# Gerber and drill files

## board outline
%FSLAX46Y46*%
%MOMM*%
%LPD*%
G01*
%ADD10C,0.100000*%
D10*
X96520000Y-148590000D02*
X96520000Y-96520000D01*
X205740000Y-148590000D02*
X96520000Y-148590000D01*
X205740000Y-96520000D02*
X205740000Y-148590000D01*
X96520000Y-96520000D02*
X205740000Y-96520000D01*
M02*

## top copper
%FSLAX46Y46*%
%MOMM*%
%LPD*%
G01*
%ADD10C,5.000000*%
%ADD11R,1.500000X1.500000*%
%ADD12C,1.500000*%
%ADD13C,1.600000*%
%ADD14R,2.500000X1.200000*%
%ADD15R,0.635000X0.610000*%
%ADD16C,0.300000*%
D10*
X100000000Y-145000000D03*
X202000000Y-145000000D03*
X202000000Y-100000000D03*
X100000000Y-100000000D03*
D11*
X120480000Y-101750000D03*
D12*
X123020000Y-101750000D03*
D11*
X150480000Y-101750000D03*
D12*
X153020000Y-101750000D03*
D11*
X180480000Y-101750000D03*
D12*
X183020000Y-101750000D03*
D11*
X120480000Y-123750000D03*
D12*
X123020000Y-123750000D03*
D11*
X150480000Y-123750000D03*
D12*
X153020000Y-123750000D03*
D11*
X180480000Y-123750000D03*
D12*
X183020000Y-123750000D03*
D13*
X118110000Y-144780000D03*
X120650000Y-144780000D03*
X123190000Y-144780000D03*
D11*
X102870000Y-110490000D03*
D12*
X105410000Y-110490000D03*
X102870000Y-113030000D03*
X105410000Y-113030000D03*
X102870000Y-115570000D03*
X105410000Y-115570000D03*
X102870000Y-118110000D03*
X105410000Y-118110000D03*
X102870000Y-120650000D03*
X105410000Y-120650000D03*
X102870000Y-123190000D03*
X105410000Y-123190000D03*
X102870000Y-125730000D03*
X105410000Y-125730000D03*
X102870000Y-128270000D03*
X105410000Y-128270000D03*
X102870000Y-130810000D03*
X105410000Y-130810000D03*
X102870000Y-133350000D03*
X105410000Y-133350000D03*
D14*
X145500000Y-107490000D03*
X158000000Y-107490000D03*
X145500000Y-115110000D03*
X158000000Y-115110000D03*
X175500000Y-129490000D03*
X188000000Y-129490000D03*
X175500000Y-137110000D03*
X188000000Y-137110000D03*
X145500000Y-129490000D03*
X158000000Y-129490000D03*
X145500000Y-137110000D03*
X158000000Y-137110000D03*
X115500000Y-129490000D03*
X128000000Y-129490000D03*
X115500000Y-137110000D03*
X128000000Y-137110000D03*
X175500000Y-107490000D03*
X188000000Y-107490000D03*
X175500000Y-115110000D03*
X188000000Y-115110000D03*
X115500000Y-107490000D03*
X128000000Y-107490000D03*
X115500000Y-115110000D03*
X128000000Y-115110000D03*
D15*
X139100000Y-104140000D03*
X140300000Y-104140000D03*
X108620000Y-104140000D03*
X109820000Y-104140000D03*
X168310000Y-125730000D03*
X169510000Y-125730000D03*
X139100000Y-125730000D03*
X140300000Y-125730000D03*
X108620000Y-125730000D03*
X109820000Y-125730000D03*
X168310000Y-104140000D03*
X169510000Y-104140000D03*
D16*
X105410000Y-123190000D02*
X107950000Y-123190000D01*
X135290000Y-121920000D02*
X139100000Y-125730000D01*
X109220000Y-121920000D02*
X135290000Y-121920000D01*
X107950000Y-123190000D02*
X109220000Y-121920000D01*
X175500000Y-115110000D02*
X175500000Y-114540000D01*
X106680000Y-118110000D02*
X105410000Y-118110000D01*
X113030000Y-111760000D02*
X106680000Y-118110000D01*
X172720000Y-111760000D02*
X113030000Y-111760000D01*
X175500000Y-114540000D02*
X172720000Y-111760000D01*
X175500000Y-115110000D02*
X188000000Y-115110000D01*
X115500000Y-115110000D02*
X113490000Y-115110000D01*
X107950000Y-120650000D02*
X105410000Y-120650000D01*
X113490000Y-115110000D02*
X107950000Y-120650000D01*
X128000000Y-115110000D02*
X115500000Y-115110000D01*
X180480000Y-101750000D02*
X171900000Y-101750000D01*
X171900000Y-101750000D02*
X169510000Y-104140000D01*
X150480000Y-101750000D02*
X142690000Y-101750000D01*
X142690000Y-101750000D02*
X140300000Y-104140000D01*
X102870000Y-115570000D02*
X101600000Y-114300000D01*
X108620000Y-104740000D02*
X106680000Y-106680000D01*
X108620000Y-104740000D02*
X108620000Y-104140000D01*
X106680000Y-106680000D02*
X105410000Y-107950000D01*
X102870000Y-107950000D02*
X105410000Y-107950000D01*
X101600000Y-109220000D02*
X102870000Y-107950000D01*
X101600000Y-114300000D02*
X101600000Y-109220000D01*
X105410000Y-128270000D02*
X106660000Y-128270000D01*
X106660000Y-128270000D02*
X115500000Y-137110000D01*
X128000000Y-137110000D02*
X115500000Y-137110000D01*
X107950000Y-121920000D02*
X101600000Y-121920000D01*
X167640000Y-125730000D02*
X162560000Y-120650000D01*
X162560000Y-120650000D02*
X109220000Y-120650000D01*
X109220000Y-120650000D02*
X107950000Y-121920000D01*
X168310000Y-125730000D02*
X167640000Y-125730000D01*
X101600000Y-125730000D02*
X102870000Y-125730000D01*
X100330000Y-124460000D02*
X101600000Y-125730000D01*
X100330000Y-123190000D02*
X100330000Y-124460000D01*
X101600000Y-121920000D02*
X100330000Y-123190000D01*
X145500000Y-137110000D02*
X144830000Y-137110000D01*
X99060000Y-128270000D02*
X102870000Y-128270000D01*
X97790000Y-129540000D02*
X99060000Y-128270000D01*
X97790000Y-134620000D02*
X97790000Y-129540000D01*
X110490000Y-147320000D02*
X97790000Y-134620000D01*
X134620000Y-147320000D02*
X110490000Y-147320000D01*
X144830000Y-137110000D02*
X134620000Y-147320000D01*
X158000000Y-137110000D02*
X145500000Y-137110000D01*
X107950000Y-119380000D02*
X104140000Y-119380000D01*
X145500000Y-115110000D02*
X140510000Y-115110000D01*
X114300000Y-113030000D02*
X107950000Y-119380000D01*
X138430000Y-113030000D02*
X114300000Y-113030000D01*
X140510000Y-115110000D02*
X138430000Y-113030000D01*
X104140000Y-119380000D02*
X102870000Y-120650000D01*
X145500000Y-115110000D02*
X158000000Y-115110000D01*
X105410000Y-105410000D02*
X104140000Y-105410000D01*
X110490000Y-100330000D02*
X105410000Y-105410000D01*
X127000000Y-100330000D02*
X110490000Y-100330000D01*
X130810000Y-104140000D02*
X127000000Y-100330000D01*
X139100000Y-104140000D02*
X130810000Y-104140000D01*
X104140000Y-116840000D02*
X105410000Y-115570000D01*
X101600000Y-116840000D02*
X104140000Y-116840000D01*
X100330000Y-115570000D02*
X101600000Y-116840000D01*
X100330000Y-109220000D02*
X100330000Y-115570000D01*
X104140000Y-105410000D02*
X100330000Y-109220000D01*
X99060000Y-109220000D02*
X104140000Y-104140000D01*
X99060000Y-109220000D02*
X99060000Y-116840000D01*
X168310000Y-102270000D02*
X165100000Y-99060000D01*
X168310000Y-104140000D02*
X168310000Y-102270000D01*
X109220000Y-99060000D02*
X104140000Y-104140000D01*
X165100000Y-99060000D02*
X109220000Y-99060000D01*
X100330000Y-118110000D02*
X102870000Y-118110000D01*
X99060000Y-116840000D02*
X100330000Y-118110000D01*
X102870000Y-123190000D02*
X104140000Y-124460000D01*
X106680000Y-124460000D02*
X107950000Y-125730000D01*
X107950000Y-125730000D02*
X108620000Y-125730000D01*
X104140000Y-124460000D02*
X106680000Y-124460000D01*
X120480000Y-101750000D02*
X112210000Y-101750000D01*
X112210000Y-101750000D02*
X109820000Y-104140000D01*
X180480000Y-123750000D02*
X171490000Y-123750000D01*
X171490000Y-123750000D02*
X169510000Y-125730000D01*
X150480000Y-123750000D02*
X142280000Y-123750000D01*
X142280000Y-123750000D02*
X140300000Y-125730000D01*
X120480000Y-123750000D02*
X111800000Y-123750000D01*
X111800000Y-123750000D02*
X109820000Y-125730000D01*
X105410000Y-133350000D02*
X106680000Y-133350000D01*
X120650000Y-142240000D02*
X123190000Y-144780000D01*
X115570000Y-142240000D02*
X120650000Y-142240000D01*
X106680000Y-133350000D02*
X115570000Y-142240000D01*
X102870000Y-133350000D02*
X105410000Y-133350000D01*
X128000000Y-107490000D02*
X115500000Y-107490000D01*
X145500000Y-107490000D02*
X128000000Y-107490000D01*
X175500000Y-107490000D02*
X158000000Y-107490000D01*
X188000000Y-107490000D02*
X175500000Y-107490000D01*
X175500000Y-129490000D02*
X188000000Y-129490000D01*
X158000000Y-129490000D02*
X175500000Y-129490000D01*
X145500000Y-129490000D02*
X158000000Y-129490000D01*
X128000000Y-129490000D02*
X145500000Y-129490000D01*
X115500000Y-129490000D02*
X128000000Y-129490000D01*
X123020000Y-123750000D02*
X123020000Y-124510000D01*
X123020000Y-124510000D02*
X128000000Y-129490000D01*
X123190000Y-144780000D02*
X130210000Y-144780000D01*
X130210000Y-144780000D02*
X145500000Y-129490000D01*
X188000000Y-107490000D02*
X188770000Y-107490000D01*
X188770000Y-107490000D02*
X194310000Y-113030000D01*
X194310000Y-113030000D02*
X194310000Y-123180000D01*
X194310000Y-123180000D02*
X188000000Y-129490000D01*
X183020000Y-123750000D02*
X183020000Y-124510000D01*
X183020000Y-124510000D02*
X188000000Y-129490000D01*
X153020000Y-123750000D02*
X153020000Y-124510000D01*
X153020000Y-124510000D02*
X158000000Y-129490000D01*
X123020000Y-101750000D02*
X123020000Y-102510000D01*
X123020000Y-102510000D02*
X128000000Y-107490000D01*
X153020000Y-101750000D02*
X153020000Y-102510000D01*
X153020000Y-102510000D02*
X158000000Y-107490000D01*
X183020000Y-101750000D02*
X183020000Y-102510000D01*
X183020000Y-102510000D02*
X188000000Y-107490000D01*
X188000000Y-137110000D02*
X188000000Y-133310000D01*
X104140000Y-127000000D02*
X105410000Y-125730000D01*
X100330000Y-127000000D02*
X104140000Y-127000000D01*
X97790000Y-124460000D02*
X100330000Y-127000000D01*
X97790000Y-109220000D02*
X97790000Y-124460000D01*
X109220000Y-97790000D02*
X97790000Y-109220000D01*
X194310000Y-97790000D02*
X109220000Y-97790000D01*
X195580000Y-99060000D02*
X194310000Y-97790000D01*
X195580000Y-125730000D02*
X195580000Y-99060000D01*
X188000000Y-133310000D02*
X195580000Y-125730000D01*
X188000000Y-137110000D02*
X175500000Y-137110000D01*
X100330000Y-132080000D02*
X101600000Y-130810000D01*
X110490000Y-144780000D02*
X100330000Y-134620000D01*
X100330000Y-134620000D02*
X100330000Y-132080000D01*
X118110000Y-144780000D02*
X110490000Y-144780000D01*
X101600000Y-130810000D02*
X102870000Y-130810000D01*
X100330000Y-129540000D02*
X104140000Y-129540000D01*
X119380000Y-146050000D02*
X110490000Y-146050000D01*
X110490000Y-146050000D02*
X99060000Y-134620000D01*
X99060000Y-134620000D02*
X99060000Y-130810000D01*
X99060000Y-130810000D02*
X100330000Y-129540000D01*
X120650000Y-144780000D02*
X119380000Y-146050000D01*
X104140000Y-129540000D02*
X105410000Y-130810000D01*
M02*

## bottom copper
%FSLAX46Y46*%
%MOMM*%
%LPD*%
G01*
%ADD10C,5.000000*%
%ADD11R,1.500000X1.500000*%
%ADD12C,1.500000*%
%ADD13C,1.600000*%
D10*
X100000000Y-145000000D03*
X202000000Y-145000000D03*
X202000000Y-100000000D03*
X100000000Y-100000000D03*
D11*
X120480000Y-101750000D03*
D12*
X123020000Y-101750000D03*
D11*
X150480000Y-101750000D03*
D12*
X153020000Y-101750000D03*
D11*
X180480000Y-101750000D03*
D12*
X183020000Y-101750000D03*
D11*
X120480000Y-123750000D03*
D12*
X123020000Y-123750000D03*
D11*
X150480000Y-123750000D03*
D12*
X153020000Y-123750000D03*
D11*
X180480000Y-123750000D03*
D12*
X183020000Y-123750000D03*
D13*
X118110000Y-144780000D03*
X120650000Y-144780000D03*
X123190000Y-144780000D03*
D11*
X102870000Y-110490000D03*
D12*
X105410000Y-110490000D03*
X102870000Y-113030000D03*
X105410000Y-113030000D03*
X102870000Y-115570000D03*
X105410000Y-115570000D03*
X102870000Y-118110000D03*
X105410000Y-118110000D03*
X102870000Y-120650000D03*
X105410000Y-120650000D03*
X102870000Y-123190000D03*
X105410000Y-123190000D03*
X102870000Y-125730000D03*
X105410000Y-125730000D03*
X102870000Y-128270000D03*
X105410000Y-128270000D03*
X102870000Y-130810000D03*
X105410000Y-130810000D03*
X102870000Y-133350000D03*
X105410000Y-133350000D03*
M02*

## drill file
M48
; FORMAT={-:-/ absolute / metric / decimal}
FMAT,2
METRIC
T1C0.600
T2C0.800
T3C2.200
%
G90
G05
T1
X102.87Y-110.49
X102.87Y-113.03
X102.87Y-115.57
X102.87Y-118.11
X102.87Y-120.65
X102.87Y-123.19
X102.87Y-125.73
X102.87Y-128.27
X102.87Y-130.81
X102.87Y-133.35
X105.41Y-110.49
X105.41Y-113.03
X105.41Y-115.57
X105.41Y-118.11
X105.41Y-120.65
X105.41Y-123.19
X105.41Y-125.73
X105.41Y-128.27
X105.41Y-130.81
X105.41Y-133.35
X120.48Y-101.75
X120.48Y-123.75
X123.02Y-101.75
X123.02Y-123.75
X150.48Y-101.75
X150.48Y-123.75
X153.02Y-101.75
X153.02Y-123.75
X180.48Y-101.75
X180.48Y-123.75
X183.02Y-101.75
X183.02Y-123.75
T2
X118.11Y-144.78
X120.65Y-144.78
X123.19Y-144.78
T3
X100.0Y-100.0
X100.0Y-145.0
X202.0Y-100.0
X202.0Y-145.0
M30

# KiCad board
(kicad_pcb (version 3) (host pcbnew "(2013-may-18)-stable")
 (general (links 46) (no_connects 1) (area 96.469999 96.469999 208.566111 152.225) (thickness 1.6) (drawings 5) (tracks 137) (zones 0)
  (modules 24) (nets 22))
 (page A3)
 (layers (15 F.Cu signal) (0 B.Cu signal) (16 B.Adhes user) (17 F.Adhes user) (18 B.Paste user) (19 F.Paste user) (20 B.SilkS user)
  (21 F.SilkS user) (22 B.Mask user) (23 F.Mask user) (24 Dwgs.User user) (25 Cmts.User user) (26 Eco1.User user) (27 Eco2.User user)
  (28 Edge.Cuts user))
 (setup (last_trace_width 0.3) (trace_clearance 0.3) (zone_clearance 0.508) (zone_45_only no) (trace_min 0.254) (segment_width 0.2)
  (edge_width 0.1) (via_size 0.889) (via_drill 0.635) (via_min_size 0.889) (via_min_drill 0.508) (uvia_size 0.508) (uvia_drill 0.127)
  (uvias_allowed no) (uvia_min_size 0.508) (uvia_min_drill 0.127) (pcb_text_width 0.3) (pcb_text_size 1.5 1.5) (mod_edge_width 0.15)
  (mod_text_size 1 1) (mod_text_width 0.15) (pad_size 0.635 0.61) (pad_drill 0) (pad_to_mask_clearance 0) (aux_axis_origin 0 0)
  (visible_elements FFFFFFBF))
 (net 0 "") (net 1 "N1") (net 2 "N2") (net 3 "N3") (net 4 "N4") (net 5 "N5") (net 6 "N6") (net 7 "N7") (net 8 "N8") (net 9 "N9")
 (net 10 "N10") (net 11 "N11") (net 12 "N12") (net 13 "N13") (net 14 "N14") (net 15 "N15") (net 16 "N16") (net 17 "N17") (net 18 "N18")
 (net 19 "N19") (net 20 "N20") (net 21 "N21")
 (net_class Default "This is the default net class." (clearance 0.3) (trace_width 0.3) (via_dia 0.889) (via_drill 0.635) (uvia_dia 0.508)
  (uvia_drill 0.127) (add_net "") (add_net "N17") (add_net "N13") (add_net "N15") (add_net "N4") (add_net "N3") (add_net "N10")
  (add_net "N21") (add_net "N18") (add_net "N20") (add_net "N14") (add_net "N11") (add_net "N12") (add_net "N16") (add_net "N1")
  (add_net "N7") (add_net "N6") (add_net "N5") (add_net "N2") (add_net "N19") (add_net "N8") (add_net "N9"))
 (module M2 (layer F.Cu) (at 100 145)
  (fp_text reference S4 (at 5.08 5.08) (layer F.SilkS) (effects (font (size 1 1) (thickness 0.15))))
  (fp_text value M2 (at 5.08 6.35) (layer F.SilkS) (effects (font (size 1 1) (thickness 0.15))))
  (pad P thru_hole circle (at 0 0) (size 5 5) (drill 2.2) (layers *.Cu *.Mask F.SilkS)))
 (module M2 (layer F.Cu) (at 202 145)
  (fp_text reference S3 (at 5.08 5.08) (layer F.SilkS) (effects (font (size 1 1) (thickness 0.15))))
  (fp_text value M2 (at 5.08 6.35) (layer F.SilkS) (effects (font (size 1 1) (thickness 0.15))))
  (pad P thru_hole circle (at 0 0) (size 5 5) (drill 2.2) (layers *.Cu *.Mask F.SilkS)))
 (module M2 (layer F.Cu) (at 202 100)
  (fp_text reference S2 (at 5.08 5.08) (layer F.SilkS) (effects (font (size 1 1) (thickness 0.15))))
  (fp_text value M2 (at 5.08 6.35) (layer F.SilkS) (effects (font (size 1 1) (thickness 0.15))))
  (pad P thru_hole circle (at 0 0) (size 5 5) (drill 2.2) (layers *.Cu *.Mask F.SilkS)))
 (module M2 (layer F.Cu) (at 100 100)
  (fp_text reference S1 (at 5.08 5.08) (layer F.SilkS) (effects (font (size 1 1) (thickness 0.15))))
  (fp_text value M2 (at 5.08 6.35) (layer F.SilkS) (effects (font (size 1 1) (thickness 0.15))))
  (pad P thru_hole circle (at 0 0) (size 5 5) (drill 2.2) (layers *.Cu *.Mask F.SilkS)))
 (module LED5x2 (layer F.Cu) (at 121.75 101.75)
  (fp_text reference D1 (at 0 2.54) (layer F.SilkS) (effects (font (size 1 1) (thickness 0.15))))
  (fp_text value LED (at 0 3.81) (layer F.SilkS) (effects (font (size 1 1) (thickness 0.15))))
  (pad 1 thru_hole rect (at -1.27 0) (size 1.5 1.5) (drill 0.6) (layers *.Cu *.Mask F.SilkS) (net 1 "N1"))
  (pad 2 thru_hole circle (at 1.27 0) (size 1.5 1.5) (drill 0.6) (layers *.Cu *.Mask F.SilkS) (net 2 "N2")))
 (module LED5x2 (layer F.Cu) (at 151.75 101.75)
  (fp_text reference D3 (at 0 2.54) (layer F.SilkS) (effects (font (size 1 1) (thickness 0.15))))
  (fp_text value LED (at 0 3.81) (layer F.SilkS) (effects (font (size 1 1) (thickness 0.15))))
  (pad 1 thru_hole rect (at -1.27 0) (size 1.5 1.5) (drill 0.6) (layers *.Cu *.Mask F.SilkS) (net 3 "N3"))
  (pad 2 thru_hole circle (at 1.27 0) (size 1.5 1.5) (drill 0.6) (layers *.Cu *.Mask F.SilkS) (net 2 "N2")))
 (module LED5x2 (layer F.Cu) (at 181.75 101.75)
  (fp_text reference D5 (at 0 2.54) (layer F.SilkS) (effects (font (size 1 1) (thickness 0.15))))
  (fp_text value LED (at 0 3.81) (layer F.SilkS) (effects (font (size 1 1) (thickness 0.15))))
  (pad 1 thru_hole rect (at -1.27 0) (size 1.5 1.5) (drill 0.6) (layers *.Cu *.Mask F.SilkS) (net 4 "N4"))
  (pad 2 thru_hole circle (at 1.27 0) (size 1.5 1.5) (drill 0.6) (layers *.Cu *.Mask F.SilkS) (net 2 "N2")))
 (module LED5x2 (layer F.Cu) (at 121.75 123.75)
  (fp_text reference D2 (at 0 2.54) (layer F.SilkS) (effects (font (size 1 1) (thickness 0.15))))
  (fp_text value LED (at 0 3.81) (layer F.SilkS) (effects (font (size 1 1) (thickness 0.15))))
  (pad 1 thru_hole rect (at -1.27 0) (size 1.5 1.5) (drill 0.6) (layers *.Cu *.Mask F.SilkS) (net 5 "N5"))
  (pad 2 thru_hole circle (at 1.27 0) (size 1.5 1.5) (drill 0.6) (layers *.Cu *.Mask F.SilkS) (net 2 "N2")))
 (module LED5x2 (layer F.Cu) (at 151.75 123.75)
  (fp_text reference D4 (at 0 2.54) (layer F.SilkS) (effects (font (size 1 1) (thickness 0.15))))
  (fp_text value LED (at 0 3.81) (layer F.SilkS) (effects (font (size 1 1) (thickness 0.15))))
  (pad 1 thru_hole rect (at -1.27 0) (size 1.5 1.5) (drill 0.6) (layers *.Cu *.Mask F.SilkS) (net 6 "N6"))
  (pad 2 thru_hole circle (at 1.27 0) (size 1.5 1.5) (drill 0.6) (layers *.Cu *.Mask F.SilkS) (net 2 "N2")))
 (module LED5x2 (layer F.Cu) (at 181.75 123.75)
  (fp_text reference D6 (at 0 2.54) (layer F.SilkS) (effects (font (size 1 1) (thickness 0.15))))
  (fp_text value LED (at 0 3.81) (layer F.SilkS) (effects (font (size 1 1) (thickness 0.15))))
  (pad 1 thru_hole rect (at -1.27 0) (size 1.5 1.5) (drill 0.6) (layers *.Cu *.Mask F.SilkS) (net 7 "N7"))
  (pad 2 thru_hole circle (at 1.27 0) (size 1.5 1.5) (drill 0.6) (layers *.Cu *.Mask F.SilkS) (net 2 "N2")))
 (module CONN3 (layer F.Cu) (at 120.65 144.78)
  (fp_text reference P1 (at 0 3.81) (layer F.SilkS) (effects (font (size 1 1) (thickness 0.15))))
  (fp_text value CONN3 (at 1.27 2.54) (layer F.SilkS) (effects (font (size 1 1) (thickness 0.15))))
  (pad 1 thru_hole circle (at -2.54 0) (size 1.6 1.6) (drill 0.8) (layers *.Cu *.Mask F.SilkS) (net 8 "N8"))
  (pad 2 thru_hole circle (at 0 0) (size 1.6 1.6) (drill 0.8) (layers *.Cu *.Mask F.SilkS) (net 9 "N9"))
  (pad 3 thru_hole circle (at 2.54 0) (size 1.6 1.6) (drill 0.8) (layers *.Cu *.Mask F.SilkS) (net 2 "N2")))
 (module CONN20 (layer F.Cu) (at 104.14 121.92)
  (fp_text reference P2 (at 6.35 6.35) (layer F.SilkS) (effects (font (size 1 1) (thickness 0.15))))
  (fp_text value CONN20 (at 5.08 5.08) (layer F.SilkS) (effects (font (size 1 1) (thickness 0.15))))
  (pad 1 thru_hole rect (at -1.27 -11.43) (size 1.5 1.5) (drill 0.6) (layers *.Cu *.Mask F.SilkS))
  (pad 2 thru_hole circle (at 1.27 -11.43) (size 1.5 1.5) (drill 0.6) (layers *.Cu *.Mask F.SilkS))
  (pad 3 thru_hole circle (at -1.27 -8.89) (size 1.5 1.5) (drill 0.6) (layers *.Cu *.Mask F.SilkS))
  (pad 4 thru_hole circle (at 1.27 -8.89) (size 1.5 1.5) (drill 0.6) (layers *.Cu *.Mask F.SilkS))
  (pad 5 thru_hole circle (at -1.27 -6.35) (size 1.5 1.5) (drill 0.6) (layers *.Cu *.Mask F.SilkS) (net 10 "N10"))
  (pad 6 thru_hole circle (at 1.27 -6.35) (size 1.5 1.5) (drill 0.6) (layers *.Cu *.Mask F.SilkS) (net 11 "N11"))
  (pad 7 thru_hole circle (at -1.27 -3.81) (size 1.5 1.5) (drill 0.6) (layers *.Cu *.Mask F.SilkS) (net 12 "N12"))
  (pad 8 thru_hole circle (at 1.27 -3.81) (size 1.5 1.5) (drill 0.6) (layers *.Cu *.Mask F.SilkS) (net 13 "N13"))
  (pad 9 thru_hole circle (at -1.27 -1.27) (size 1.5 1.5) (drill 0.6) (layers *.Cu *.Mask F.SilkS) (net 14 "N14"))
  (pad 10 thru_hole circle (at 1.27 -1.27) (size 1.5 1.5) (drill 0.6) (layers *.Cu *.Mask F.SilkS) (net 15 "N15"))
  (pad 11 thru_hole circle (at -1.27 1.27) (size 1.5 1.5) (drill 0.6) (layers *.Cu *.Mask F.SilkS) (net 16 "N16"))
  (pad 12 thru_hole circle (at 1.27 1.27) (size 1.5 1.5) (drill 0.6) (layers *.Cu *.Mask F.SilkS) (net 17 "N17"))
  (pad 13 thru_hole circle (at -1.27 3.81) (size 1.5 1.5) (drill 0.6) (layers *.Cu *.Mask F.SilkS) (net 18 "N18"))
  (pad 14 thru_hole circle (at 1.27 3.81) (size 1.5 1.5) (drill 0.6) (layers *.Cu *.Mask F.SilkS) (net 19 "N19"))
  (pad 15 thru_hole circle (at -1.27 6.35) (size 1.5 1.5) (drill 0.6) (layers *.Cu *.Mask F.SilkS) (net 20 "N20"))
  (pad 16 thru_hole circle (at 1.27 6.35) (size 1.5 1.5) (drill 0.6) (layers *.Cu *.Mask F.SilkS) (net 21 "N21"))
  (pad 17 thru_hole circle (at -1.27 8.89) (size 1.5 1.5) (drill 0.6) (layers *.Cu *.Mask F.SilkS) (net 8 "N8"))
  (pad 18 thru_hole circle (at 1.27 8.89) (size 1.5 1.5) (drill 0.6) (layers *.Cu *.Mask F.SilkS) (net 9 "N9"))
  (pad 19 thru_hole circle (at -1.27 11.43) (size 1.5 1.5) (drill 0.6) (layers *.Cu *.Mask F.SilkS) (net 2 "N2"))
  (pad 20 thru_hole circle (at 1.27 11.43) (size 1.5 1.5) (drill 0.6) (layers *.Cu *.Mask F.SilkS) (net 2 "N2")))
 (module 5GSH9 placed (layer F.Cu) (at 151.75 111.3)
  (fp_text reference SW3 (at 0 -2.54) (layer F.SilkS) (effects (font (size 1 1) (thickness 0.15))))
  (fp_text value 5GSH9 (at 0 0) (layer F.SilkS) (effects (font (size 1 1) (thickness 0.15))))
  (pad 2 smd rect (at -6.25 -3.81) (size 2.5 1.2) (layers F.Cu F.Paste F.Mask) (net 2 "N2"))
  (pad 1 smd rect (at 6.25 -3.81) (size 2.5 1.2) (layers F.Cu F.Paste F.Mask) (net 2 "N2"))
  (pad 4 smd rect (at -6.25 3.81) (size 2.5 1.2) (layers F.Cu F.Paste F.Mask) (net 14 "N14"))
  (pad 3 smd rect (at 6.25 3.81) (size 2.5 1.2) (layers F.Cu F.Paste F.Mask) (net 14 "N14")))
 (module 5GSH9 (layer F.Cu) (at 181.75 133.3)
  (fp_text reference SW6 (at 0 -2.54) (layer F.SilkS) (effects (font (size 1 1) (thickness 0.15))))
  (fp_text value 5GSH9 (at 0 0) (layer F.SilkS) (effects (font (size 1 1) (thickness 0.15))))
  (pad 2 smd rect (at -6.25 -3.81) (size 2.5 1.2) (layers F.Cu F.Paste F.Mask) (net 2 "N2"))
  (pad 1 smd rect (at 6.25 -3.81) (size 2.5 1.2) (layers F.Cu F.Paste F.Mask) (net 2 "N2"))
  (pad 4 smd rect (at -6.25 3.81) (size 2.5 1.2) (layers F.Cu F.Paste F.Mask) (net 19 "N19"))
  (pad 3 smd rect (at 6.25 3.81) (size 2.5 1.2) (layers F.Cu F.Paste F.Mask) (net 19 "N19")))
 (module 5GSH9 (layer F.Cu) (at 151.75 133.3)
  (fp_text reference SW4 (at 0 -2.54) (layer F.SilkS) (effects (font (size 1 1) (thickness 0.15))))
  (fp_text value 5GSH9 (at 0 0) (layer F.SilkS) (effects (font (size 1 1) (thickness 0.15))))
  (pad 2 smd rect (at -6.25 -3.81) (size 2.5 1.2) (layers F.Cu F.Paste F.Mask) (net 2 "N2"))
  (pad 1 smd rect (at 6.25 -3.81) (size 2.5 1.2) (layers F.Cu F.Paste F.Mask) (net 2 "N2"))
  (pad 4 smd rect (at -6.25 3.81) (size 2.5 1.2) (layers F.Cu F.Paste F.Mask) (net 20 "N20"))
  (pad 3 smd rect (at 6.25 3.81) (size 2.5 1.2) (layers F.Cu F.Paste F.Mask) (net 20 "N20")))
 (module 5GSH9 (layer F.Cu) (at 121.75 133.3)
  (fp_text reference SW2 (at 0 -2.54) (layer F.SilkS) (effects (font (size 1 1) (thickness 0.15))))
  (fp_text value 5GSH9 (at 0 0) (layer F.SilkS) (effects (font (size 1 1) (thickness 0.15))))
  (pad 2 smd rect (at -6.25 -3.81) (size 2.5 1.2) (layers F.Cu F.Paste F.Mask) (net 2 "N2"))
  (pad 1 smd rect (at 6.25 -3.81) (size 2.5 1.2) (layers F.Cu F.Paste F.Mask) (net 2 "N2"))
  (pad 4 smd rect (at -6.25 3.81) (size 2.5 1.2) (layers F.Cu F.Paste F.Mask) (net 21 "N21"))
  (pad 3 smd rect (at 6.25 3.81) (size 2.5 1.2) (layers F.Cu F.Paste F.Mask) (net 21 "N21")))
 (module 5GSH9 (layer F.Cu) (at 181.75 111.3)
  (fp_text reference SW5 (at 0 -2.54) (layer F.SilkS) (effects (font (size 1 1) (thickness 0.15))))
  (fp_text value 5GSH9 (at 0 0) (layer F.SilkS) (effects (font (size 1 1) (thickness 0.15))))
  (pad 2 smd rect (at -6.25 -3.81) (size 2.5 1.2) (layers F.Cu F.Paste F.Mask) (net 2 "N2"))
  (pad 1 smd rect (at 6.25 -3.81) (size 2.5 1.2) (layers F.Cu F.Paste F.Mask) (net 2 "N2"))
  (pad 4 smd rect (at -6.25 3.81) (size 2.5 1.2) (layers F.Cu F.Paste F.Mask) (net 13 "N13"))
  (pad 3 smd rect (at 6.25 3.81) (size 2.5 1.2) (layers F.Cu F.Paste F.Mask) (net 13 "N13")))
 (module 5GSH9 (layer F.Cu) (at 121.75 111.3)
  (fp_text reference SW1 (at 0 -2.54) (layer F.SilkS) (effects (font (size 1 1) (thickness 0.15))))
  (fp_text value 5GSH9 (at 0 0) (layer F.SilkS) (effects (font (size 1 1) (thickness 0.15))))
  (pad 2 smd rect (at -6.25 -3.81) (size 2.5 1.2) (layers F.Cu F.Paste F.Mask) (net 2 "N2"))
  (pad 1 smd rect (at 6.25 -3.81) (size 2.5 1.2) (layers F.Cu F.Paste F.Mask) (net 2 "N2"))
  (pad 4 smd rect (at -6.25 3.81) (size 2.5 1.2) (layers F.Cu F.Paste F.Mask) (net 15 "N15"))
  (pad 3 smd rect (at 6.25 3.81) (size 2.5 1.2) (layers F.Cu F.Paste F.Mask) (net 15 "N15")))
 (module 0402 (layer F.Cu) (at 139.7 104.14)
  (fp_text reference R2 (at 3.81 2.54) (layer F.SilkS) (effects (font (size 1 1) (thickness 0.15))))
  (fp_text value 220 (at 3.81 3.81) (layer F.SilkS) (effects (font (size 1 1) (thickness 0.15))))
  (pad 1 smd rect (at -0.6 0) (size 0.635 0.61) (layers F.Cu F.Paste F.Mask) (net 11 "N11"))
  (pad 2 smd rect (at 0.6 0) (size 0.635 0.61) (layers F.Cu F.Paste F.Mask) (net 3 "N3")))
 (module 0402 (layer F.Cu) (at 109.22 104.14)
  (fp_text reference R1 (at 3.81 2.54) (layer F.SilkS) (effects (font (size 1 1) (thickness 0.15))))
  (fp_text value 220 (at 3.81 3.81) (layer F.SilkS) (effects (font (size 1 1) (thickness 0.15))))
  (pad 1 smd rect (at -0.6 0) (size 0.635 0.61) (layers F.Cu F.Paste F.Mask) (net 10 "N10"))
  (pad 2 smd rect (at 0.6 0) (size 0.635 0.61) (layers F.Cu F.Paste F.Mask) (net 1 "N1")))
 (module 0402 (layer F.Cu) (at 168.91 125.73)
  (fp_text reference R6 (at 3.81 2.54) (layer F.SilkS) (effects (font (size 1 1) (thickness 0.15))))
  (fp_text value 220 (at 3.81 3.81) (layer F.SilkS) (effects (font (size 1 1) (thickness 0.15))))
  (pad 1 smd rect (at -0.6 0) (size 0.635 0.61) (layers F.Cu F.Paste F.Mask) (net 18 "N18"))
  (pad 2 smd rect (at 0.6 0) (size 0.635 0.61) (layers F.Cu F.Paste F.Mask) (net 7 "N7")))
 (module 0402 (layer F.Cu) (at 139.7 125.73)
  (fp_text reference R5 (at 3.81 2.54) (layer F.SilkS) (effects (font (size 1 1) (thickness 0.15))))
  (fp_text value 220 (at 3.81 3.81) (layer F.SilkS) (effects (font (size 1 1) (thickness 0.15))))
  (pad 1 smd rect (at -0.6 0) (size 0.635 0.61) (layers F.Cu F.Paste F.Mask) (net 17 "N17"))
  (pad 2 smd rect (at 0.6 0) (size 0.635 0.61) (layers F.Cu F.Paste F.Mask) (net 6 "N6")))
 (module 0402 (layer F.Cu) (at 109.22 125.73)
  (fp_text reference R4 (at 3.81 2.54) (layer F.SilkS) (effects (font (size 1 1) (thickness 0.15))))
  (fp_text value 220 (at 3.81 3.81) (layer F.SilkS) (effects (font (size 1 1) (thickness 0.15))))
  (pad 1 smd rect (at -0.6 0) (size 0.635 0.61) (layers F.Cu F.Paste F.Mask) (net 16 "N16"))
  (pad 2 smd rect (at 0.6 0) (size 0.635 0.61) (layers F.Cu F.Paste F.Mask) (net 5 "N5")))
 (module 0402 (layer F.Cu) (at 168.91 104.14)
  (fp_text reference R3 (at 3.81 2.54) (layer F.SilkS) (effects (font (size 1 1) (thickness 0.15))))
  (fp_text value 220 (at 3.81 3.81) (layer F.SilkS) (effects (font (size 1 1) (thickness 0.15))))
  (pad 1 smd rect (at -0.6 0) (size 0.635 0.61) (layers F.Cu F.Paste F.Mask) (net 12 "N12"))
  (pad 2 smd rect (at 0.6 0) (size 0.635 0.61) (layers F.Cu F.Paste F.Mask) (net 4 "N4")))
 (gr_line (start 96.52 148.59) (end 96.52 96.52) (angle 90) (layer Edge.Cuts) (width 0.1))
 (gr_line (start 205.74 148.59) (end 96.52 148.59) (angle 90) (layer Edge.Cuts) (width 0.1))
 (gr_line (start 205.74 96.52) (end 205.74 148.59) (angle 90) (layer Edge.Cuts) (width 0.1))
 (gr_line (start 96.52 96.52) (end 205.74 96.52) (angle 90) (layer Edge.Cuts) (width 0.1))
 (segment (start 105.41 123.19) (end 107.95 123.19) (width 0.3) (layer F.Cu) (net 17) (status 10))
 (segment (start 135.29 121.92) (end 139.1 125.73) (width 0.3) (layer F.Cu) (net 17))
 (segment (start 109.22 121.92) (end 135.29 121.92) (width 0.3) (layer F.Cu) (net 17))
 (segment (start 107.95 123.19) (end 109.22 121.92) (width 0.3) (layer F.Cu) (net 17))
 (segment (start 175.5 115.11) (end 175.5 114.54) (width 0.3) (layer F.Cu) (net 13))
 (segment (start 106.68 118.11) (end 105.41 118.11) (width 0.3) (layer F.Cu) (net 13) (status 20))
 (segment (start 113.03 111.76) (end 106.68 118.11) (width 0.3) (layer F.Cu) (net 13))
 (segment (start 172.72 111.76) (end 113.03 111.76) (width 0.3) (layer F.Cu) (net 13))
 (segment (start 175.5 114.54) (end 172.72 111.76) (width 0.3) (layer F.Cu) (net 13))
 (segment (start 175.5 115.11) (end 188 115.11) (width 0.3) (layer F.Cu) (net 13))
 (segment (start 115.5 115.11) (end 113.49 115.11) (width 0.3) (layer F.Cu) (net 15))
 (segment (start 107.95 120.65) (end 105.41 120.65) (width 0.3) (layer F.Cu) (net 15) (status 20))
 (segment (start 113.49 115.11) (end 107.95 120.65) (width 0.3) (layer F.Cu) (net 15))
 (segment (start 128 115.11) (end 115.5 115.11) (width 0.3) (layer F.Cu) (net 15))
 (segment (start 180.48 101.75) (end 171.9 101.75) (width 0.3) (layer F.Cu) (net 4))
 (segment (start 171.9 101.75) (end 169.51 104.14) (width 0.3) (layer F.Cu) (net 4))
 (segment (start 150.48 101.75) (end 142.69 101.75) (width 0.3) (layer F.Cu) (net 3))
 (segment (start 142.69 101.75) (end 140.3 104.14) (width 0.3) (layer F.Cu) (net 3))
 (segment (start 102.87 115.57) (end 101.6 114.3) (width 0.3) (layer F.Cu) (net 10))
 (segment (start 108.62 104.74) (end 106.68 106.68) (width 0.3) (layer F.Cu) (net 10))
 (segment (start 108.62 104.74) (end 108.62 104.14) (width 0.3) (layer F.Cu) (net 10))
 (segment (start 106.68 106.68) (end 105.41 107.95) (width 0.3) (layer F.Cu) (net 10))
 (segment (start 102.87 107.95) (end 105.41 107.95) (width 0.3) (layer F.Cu) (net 10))
 (segment (start 101.6 109.22) (end 102.87 107.95) (width 0.3) (layer F.Cu) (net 10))
 (segment (start 101.6 114.3) (end 101.6 109.22) (width 0.3) (layer F.Cu) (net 10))
 (segment (start 105.41 128.27) (end 106.66 128.27) (width 0.3) (layer F.Cu) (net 21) (status 10))
 (segment (start 106.66 128.27) (end 115.5 137.11) (width 0.3) (layer F.Cu) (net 21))
 (segment (start 128 137.11) (end 115.5 137.11) (width 0.3) (layer F.Cu) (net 21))
 (segment (start 107.95 121.92) (end 101.6 121.92) (width 0.3) (layer F.Cu) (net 18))
 (segment (start 167.64 125.73) (end 162.56 120.65) (width 0.3) (layer F.Cu) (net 18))
 (segment (start 162.56 120.65) (end 109.22 120.65) (width 0.3) (layer F.Cu) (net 18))
 (segment (start 109.22 120.65) (end 107.95 121.92) (width 0.3) (layer F.Cu) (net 18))
 (segment (start 168.31 125.73) (end 167.64 125.73) (width 0.3) (layer F.Cu) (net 18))
 (segment (start 101.6 125.73) (end 102.87 125.73) (width 0.3) (layer F.Cu) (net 18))
 (segment (start 100.33 124.46) (end 101.6 125.73) (width 0.3) (layer F.Cu) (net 18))
 (segment (start 100.33 123.19) (end 100.33 124.46) (width 0.3) (layer F.Cu) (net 18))
 (segment (start 101.6 121.92) (end 100.33 123.19) (width 0.3) (layer F.Cu) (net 18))
 (segment (start 145.5 137.11) (end 144.83 137.11) (width 0.3) (layer F.Cu) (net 20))
 (segment (start 99.06 128.27) (end 102.87 128.27) (width 0.3) (layer F.Cu) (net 20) (status 20))
 (segment (start 97.79 129.54) (end 99.06 128.27) (width 0.3) (layer F.Cu) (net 20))
 (segment (start 97.79 134.62) (end 97.79 129.54) (width 0.3) (layer F.Cu) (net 20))
 (segment (start 110.49 147.32) (end 97.79 134.62) (width 0.3) (layer F.Cu) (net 20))
 (segment (start 134.62 147.32) (end 110.49 147.32) (width 0.3) (layer F.Cu) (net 20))
 (segment (start 144.83 137.11) (end 134.62 147.32) (width 0.3) (layer F.Cu) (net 20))
 (segment (start 158 137.11) (end 145.5 137.11) (width 0.3) (layer F.Cu) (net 20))
 (segment (start 107.95 119.38) (end 104.14 119.38) (width 0.3) (layer F.Cu) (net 14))
 (segment (start 145.5 115.11) (end 140.51 115.11) (width 0.3) (layer F.Cu) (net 14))
 (segment (start 114.3 113.03) (end 107.95 119.38) (width 0.3) (layer F.Cu) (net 14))
 (segment (start 138.43 113.03) (end 114.3 113.03) (width 0.3) (layer F.Cu) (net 14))
 (segment (start 140.51 115.11) (end 138.43 113.03) (width 0.3) (layer F.Cu) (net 14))
 (segment (start 104.14 119.38) (end 102.87 120.65) (width 0.3) (layer F.Cu) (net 14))
 (segment (start 145.5 115.11) (end 158 115.11) (width 0.3) (layer F.Cu) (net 14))
 (segment (start 105.41 105.41) (end 104.14 105.41) (width 0.3) (layer F.Cu) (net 11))
 (segment (start 110.49 100.33) (end 105.41 105.41) (width 0.3) (layer F.Cu) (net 11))
 (segment (start 127 100.33) (end 110.49 100.33) (width 0.3) (layer F.Cu) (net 11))
 (segment (start 130.81 104.14) (end 127 100.33) (width 0.3) (layer F.Cu) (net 11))
 (segment (start 139.1 104.14) (end 130.81 104.14) (width 0.3) (layer F.Cu) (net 11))
 (segment (start 104.14 116.84) (end 105.41 115.57) (width 0.3) (layer F.Cu) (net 11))
 (segment (start 101.6 116.84) (end 104.14 116.84) (width 0.3) (layer F.Cu) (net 11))
 (segment (start 100.33 115.57) (end 101.6 116.84) (width 0.3) (layer F.Cu) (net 11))
 (segment (start 100.33 109.22) (end 100.33 115.57) (width 0.3) (layer F.Cu) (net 11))
 (segment (start 104.14 105.41) (end 100.33 109.22) (width 0.3) (layer F.Cu) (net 11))
 (segment (start 99.06 109.22) (end 104.14 104.14) (width 0.3) (layer F.Cu) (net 12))
 (segment (start 99.06 109.22) (end 99.06 116.84) (width 0.3) (layer F.Cu) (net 12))
 (segment (start 168.31 102.27) (end 165.1 99.06) (width 0.3) (layer F.Cu) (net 12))
 (segment (start 168.31 104.14) (end 168.31 102.27) (width 0.3) (layer F.Cu) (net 12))
 (segment (start 109.22 99.06) (end 104.14 104.14) (width 0.3) (layer F.Cu) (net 12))
 (segment (start 165.1 99.06) (end 109.22 99.06) (width 0.3) (layer F.Cu) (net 12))
 (segment (start 100.33 118.11) (end 102.87 118.11) (width 0.3) (layer F.Cu) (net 12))
 (segment (start 99.06 116.84) (end 100.33 118.11) (width 0.3) (layer F.Cu) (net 12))
 (segment (start 102.87 123.19) (end 104.14 124.46) (width 0.3) (layer F.Cu) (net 16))
 (segment (start 106.68 124.46) (end 107.95 125.73) (width 0.3) (layer F.Cu) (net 16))
 (segment (start 107.95 125.73) (end 108.62 125.73) (width 0.3) (layer F.Cu) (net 16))
 (segment (start 104.14 124.46) (end 106.68 124.46) (width 0.3) (layer F.Cu) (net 16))
 (segment (start 120.48 101.75) (end 112.21 101.75) (width 0.3) (layer F.Cu) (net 1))
 (segment (start 112.21 101.75) (end 109.82 104.14) (width 0.3) (layer F.Cu) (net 1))
 (segment (start 180.48 123.75) (end 171.49 123.75) (width 0.3) (layer F.Cu) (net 7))
 (segment (start 171.49 123.75) (end 169.51 125.73) (width 0.3) (layer F.Cu) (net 7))
 (segment (start 150.48 123.75) (end 142.28 123.75) (width 0.3) (layer F.Cu) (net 6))
 (segment (start 142.28 123.75) (end 140.3 125.73) (width 0.3) (layer F.Cu) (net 6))
 (segment (start 120.48 123.75) (end 111.8 123.75) (width 0.3) (layer F.Cu) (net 5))
 (segment (start 111.8 123.75) (end 109.82 125.73) (width 0.3) (layer F.Cu) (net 5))
 (segment (start 105.41 133.35) (end 106.68 133.35) (width 0.3) (layer F.Cu) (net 2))
 (segment (start 120.65 142.24) (end 123.19 144.78) (width 0.3) (layer F.Cu) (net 2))
 (segment (start 115.57 142.24) (end 120.65 142.24) (width 0.3) (layer F.Cu) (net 2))
 (segment (start 106.68 133.35) (end 115.57 142.24) (width 0.3) (layer F.Cu) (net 2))
 (segment (start 102.87 133.35) (end 105.41 133.35) (width 0.3) (layer F.Cu) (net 2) (status 30))
 (segment (start 128 107.49) (end 115.5 107.49) (width 0.3) (layer F.Cu) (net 2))
 (segment (start 145.5 107.49) (end 128 107.49) (width 0.3) (layer F.Cu) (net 2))
 (segment (start 175.5 107.49) (end 158 107.49) (width 0.3) (layer F.Cu) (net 2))
 (segment (start 188 107.49) (end 175.5 107.49) (width 0.3) (layer F.Cu) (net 2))
 (segment (start 175.5 129.49) (end 188 129.49) (width 0.3) (layer F.Cu) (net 2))
 (segment (start 158 129.49) (end 175.5 129.49) (width 0.3) (layer F.Cu) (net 2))
 (segment (start 145.5 129.49) (end 158 129.49) (width 0.3) (layer F.Cu) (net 2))
 (segment (start 128 129.49) (end 145.5 129.49) (width 0.3) (layer F.Cu) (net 2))
 (segment (start 115.5 129.49) (end 128 129.49) (width 0.3) (layer F.Cu) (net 2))
 (segment (start 123.02 123.75) (end 123.02 124.51) (width 0.3) (layer F.Cu) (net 2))
 (segment (start 123.02 124.51) (end 128 129.49) (width 0.3) (layer F.Cu) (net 2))
 (segment (start 123.19 144.78) (end 130.21 144.78) (width 0.3) (layer F.Cu) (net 2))
 (segment (start 130.21 144.78) (end 145.5 129.49) (width 0.3) (layer F.Cu) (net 2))
 (segment (start 188 107.49) (end 188.77 107.49) (width 0.3) (layer F.Cu) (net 2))
 (segment (start 188.77 107.49) (end 194.31 113.03) (width 0.3) (layer F.Cu) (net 2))
 (segment (start 194.31 113.03) (end 194.31 123.18) (width 0.3) (layer F.Cu) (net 2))
 (segment (start 194.31 123.18) (end 188 129.49) (width 0.3) (layer F.Cu) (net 2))
 (segment (start 183.02 123.75) (end 183.02 124.51) (width 0.3) (layer F.Cu) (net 2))
 (segment (start 183.02 124.51) (end 188 129.49) (width 0.3) (layer F.Cu) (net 2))
 (segment (start 153.02 123.75) (end 153.02 124.51) (width 0.3) (layer F.Cu) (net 2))
 (segment (start 153.02 124.51) (end 158 129.49) (width 0.3) (layer F.Cu) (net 2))
 (segment (start 123.02 101.75) (end 123.02 102.51) (width 0.3) (layer F.Cu) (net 2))
 (segment (start 123.02 102.51) (end 128 107.49) (width 0.3) (layer F.Cu) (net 2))
 (segment (start 153.02 101.75) (end 153.02 102.51) (width 0.3) (layer F.Cu) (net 2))
 (segment (start 153.02 102.51) (end 158 107.49) (width 0.3) (layer F.Cu) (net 2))
 (segment (start 183.02 101.75) (end 183.02 102.51) (width 0.3) (layer F.Cu) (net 2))
 (segment (start 183.02 102.51) (end 188 107.49) (width 0.3) (layer F.Cu) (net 2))
 (segment (start 188 137.11) (end 188 133.31) (width 0.3) (layer F.Cu) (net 19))
 (segment (start 104.14 127) (end 105.41 125.73) (width 0.3) (layer F.Cu) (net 19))
 (segment (start 100.33 127) (end 104.14 127) (width 0.3) (layer F.Cu) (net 19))
 (segment (start 97.79 124.46) (end 100.33 127) (width 0.3) (layer F.Cu) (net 19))
 (segment (start 97.79 109.22) (end 97.79 124.46) (width 0.3) (layer F.Cu) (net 19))
 (segment (start 109.22 97.79) (end 97.79 109.22) (width 0.3) (layer F.Cu) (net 19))
 (segment (start 194.31 97.79) (end 109.22 97.79) (width 0.3) (layer F.Cu) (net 19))
 (segment (start 195.58 99.06) (end 194.31 97.79) (width 0.3) (layer F.Cu) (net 19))
 (segment (start 195.58 125.73) (end 195.58 99.06) (width 0.3) (layer F.Cu) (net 19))
 (segment (start 188 133.31) (end 195.58 125.73) (width 0.3) (layer F.Cu) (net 19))
 (segment (start 188 137.11) (end 175.5 137.11) (width 0.3) (layer F.Cu) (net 19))
 (segment (start 100.33 132.08) (end 101.6 130.81) (width 0.3) (layer F.Cu) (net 8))
 (segment (start 110.49 144.78) (end 100.33 134.62) (width 0.3) (layer F.Cu) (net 8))
 (segment (start 100.33 134.62) (end 100.33 132.08) (width 0.3) (layer F.Cu) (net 8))
 (segment (start 118.11 144.78) (end 110.49 144.78) (width 0.3) (layer F.Cu) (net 8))
 (segment (start 101.6 130.81) (end 102.87 130.81) (width 0.3) (layer F.Cu) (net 8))
 (segment (start 100.33 129.54) (end 104.14 129.54) (width 0.3) (layer F.Cu) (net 9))
 (segment (start 119.38 146.05) (end 110.49 146.05) (width 0.3) (layer F.Cu) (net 9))
 (segment (start 110.49 146.05) (end 99.06 134.62) (width 0.3) (layer F.Cu) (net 9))
 (segment (start 99.06 134.62) (end 99.06 130.81) (width 0.3) (layer F.Cu) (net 9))
 (segment (start 99.06 130.81) (end 100.33 129.54) (width 0.3) (layer F.Cu) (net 9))
 (segment (start 120.65 144.78) (end 119.38 146.05) (width 0.3) (layer F.Cu) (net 9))
 (segment (start 104.14 129.54) (end 105.41 130.81) (width 0.3) (layer F.Cu) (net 9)))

